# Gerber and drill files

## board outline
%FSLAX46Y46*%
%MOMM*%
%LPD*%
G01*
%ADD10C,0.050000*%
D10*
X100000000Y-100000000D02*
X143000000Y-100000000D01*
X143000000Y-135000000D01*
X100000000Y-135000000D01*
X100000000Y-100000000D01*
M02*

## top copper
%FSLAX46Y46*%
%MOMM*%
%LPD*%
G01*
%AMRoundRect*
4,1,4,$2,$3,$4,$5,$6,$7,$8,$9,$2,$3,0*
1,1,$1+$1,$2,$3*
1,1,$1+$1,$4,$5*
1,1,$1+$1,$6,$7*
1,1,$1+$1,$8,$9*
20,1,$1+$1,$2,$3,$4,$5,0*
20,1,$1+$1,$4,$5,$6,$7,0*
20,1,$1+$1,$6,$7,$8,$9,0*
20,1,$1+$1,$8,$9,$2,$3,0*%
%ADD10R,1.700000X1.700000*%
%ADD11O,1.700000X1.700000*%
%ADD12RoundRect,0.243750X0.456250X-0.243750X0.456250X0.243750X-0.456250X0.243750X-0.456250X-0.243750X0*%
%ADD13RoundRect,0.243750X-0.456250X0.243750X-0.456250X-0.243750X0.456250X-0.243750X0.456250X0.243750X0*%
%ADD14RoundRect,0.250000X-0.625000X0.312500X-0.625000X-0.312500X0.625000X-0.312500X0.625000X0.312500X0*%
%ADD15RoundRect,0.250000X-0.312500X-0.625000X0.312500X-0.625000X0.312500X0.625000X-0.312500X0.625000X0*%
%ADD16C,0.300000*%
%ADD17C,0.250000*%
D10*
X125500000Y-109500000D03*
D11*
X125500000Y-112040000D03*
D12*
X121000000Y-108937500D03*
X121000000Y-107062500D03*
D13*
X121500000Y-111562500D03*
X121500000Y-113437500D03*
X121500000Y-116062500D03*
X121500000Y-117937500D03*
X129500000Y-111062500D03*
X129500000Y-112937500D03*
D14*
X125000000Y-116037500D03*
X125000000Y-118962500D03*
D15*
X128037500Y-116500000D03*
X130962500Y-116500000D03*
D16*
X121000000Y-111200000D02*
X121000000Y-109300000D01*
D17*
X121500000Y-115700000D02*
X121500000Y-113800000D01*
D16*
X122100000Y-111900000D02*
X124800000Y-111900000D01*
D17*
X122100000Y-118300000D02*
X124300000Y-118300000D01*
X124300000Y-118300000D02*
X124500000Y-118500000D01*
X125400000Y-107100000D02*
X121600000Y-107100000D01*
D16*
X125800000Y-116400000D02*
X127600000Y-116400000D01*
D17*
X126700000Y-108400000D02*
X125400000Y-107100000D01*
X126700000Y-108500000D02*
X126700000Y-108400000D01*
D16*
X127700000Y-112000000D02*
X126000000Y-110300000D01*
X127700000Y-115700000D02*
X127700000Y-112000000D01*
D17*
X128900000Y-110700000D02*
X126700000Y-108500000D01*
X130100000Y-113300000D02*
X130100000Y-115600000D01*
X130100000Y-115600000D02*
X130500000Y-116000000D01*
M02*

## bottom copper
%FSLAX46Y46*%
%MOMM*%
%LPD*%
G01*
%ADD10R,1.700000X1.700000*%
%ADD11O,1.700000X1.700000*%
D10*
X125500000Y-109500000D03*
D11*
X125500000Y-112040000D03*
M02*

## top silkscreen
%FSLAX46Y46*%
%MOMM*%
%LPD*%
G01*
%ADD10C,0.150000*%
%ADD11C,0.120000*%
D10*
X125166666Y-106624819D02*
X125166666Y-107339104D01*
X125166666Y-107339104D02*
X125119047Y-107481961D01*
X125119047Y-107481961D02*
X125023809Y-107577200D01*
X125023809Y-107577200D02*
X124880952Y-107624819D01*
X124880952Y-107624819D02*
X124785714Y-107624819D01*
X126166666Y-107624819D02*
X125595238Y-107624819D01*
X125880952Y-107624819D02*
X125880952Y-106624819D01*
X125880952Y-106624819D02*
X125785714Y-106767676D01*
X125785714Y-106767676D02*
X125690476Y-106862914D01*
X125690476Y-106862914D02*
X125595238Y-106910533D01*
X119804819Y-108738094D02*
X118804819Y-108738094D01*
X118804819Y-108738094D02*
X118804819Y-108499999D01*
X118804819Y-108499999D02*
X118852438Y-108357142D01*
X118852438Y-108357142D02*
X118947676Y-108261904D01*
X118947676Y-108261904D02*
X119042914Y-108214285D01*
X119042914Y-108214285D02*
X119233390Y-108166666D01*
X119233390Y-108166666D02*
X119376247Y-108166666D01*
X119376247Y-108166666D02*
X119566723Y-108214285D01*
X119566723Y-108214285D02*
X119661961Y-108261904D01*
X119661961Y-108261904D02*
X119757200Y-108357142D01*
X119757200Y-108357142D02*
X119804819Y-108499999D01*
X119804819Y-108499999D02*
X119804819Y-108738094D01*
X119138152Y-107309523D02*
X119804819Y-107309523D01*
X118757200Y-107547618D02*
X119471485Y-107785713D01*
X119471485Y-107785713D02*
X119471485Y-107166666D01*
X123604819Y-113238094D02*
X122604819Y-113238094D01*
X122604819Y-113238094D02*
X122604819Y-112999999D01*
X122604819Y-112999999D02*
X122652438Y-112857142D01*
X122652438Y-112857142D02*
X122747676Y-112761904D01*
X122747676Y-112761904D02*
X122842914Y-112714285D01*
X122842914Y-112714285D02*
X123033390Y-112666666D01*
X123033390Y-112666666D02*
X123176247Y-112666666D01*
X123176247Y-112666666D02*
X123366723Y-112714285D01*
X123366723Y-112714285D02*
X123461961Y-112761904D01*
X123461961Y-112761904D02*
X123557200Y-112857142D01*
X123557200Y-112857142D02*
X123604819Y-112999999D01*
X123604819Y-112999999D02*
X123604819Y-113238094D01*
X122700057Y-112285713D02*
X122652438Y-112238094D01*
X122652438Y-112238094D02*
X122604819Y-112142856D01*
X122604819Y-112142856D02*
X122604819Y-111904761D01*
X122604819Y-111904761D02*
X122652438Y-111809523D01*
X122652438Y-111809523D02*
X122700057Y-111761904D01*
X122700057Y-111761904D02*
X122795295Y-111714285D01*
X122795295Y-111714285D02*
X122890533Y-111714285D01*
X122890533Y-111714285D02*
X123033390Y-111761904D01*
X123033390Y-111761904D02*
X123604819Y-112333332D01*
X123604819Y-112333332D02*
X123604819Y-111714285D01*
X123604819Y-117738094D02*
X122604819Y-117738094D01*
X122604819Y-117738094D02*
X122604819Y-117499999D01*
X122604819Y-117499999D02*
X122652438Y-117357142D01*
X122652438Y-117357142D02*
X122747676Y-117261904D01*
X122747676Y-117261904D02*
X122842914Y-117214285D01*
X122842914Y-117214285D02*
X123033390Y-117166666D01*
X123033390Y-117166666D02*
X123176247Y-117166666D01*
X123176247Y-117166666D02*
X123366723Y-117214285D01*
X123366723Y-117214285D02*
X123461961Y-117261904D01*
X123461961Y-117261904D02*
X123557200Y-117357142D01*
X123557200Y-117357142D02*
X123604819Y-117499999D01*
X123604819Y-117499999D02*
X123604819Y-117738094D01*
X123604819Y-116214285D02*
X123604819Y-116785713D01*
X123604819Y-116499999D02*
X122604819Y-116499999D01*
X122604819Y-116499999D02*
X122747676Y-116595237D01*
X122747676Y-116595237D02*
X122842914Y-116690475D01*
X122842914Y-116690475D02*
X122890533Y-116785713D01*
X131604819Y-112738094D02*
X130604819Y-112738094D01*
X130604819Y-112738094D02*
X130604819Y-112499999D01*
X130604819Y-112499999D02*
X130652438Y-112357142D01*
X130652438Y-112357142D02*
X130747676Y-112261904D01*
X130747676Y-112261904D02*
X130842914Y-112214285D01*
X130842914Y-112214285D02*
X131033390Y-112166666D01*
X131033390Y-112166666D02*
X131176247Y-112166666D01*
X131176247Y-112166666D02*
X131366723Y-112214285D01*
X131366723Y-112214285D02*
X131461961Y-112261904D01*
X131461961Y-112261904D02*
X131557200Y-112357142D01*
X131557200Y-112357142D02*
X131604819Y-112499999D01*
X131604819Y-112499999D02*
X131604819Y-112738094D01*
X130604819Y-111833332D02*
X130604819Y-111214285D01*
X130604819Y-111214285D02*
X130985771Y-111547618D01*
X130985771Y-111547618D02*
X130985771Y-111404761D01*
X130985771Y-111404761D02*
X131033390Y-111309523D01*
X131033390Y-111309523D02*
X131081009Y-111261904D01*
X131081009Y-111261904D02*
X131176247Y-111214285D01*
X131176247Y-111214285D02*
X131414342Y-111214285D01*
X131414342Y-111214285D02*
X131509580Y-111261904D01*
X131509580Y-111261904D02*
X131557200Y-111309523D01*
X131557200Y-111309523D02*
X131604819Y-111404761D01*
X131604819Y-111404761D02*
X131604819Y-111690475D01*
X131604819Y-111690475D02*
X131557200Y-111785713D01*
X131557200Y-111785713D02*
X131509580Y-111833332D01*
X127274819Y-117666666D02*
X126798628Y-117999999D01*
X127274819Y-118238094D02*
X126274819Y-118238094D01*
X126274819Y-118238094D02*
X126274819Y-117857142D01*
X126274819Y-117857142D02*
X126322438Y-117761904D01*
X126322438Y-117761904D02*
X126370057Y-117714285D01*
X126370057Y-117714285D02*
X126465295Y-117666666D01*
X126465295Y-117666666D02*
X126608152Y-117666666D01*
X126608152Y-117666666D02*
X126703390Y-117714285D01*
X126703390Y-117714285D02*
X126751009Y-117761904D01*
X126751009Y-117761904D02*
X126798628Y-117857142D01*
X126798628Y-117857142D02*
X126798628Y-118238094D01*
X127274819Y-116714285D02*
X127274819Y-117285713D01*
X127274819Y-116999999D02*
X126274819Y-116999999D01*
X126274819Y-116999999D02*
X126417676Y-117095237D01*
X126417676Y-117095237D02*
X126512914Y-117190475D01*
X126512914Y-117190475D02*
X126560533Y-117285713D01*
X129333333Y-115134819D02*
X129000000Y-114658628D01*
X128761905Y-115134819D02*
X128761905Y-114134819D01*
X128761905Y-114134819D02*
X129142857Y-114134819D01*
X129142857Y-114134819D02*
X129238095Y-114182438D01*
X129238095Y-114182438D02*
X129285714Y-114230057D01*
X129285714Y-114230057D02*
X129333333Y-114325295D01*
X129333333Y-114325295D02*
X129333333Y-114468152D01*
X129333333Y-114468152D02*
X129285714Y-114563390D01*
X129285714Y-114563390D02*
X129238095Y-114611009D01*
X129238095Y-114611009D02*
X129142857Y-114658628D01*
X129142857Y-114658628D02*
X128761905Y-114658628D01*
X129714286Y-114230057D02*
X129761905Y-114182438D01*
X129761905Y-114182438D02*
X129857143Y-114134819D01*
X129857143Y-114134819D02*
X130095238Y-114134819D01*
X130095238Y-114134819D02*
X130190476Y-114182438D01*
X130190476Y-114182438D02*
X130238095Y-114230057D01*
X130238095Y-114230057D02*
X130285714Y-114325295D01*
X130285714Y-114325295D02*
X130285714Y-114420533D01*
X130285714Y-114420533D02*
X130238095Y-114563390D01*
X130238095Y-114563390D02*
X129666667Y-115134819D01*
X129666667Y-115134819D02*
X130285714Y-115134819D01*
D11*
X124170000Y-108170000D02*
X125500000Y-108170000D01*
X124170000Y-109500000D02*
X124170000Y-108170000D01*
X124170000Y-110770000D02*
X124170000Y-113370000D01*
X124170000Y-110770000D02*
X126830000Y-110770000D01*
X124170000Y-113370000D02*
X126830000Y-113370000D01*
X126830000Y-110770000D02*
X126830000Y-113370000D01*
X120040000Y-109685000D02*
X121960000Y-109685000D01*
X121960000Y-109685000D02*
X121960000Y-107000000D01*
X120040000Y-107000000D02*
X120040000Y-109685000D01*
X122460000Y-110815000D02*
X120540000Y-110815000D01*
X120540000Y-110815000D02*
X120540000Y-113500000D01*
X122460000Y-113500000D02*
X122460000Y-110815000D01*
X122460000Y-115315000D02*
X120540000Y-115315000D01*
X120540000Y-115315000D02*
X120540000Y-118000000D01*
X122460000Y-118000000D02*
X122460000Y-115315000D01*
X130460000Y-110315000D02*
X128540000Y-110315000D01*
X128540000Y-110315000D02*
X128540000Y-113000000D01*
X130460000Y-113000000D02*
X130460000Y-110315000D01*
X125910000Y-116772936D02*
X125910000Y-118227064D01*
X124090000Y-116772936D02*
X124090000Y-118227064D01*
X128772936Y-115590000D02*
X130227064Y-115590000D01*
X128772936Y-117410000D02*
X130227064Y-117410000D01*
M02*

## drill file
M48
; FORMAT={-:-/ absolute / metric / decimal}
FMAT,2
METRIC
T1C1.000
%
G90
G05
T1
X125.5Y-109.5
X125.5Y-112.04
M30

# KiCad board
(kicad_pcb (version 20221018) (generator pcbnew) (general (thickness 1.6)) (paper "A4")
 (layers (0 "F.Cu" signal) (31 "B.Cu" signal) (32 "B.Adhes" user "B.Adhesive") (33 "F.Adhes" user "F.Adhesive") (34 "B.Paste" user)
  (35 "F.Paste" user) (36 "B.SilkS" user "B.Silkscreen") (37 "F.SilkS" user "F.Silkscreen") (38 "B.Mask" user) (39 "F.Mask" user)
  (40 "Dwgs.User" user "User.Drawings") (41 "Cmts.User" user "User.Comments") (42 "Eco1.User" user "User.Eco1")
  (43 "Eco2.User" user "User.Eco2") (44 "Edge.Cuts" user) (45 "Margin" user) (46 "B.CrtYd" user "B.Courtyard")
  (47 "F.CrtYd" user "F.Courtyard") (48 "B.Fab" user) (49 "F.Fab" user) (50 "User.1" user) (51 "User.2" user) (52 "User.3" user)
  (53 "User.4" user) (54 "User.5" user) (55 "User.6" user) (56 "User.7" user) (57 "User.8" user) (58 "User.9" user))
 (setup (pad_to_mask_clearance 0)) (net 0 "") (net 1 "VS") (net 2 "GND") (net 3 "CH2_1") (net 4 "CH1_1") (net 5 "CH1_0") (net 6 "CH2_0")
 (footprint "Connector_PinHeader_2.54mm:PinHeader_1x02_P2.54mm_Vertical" (layer "F.Cu") (at 125.5 109.5)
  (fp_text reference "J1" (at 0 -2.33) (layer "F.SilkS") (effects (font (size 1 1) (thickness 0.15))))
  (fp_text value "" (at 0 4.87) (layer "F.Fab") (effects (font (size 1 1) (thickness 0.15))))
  (fp_line (start -1.33 -1.33) (end 0 -1.33) (stroke (width 0.12) (type solid)) (layer "F.SilkS"))
  (fp_line (start -1.33 0) (end -1.33 -1.33) (stroke (width 0.12) (type solid)) (layer "F.SilkS"))
  (fp_line (start -1.33 1.27) (end -1.33 3.87) (stroke (width 0.12) (type solid)) (layer "F.SilkS"))
  (fp_line (start -1.33 1.27) (end 1.33 1.27) (stroke (width 0.12) (type solid)) (layer "F.SilkS"))
  (fp_line (start -1.33 3.87) (end 1.33 3.87) (stroke (width 0.12) (type solid)) (layer "F.SilkS"))
  (fp_line (start 1.33 1.27) (end 1.33 3.87) (stroke (width 0.12) (type solid)) (layer "F.SilkS"))
  (pad "1" thru_hole rect (at 0 0) (size 1.7 1.7) (drill 1) (layers "*.Cu" "*.Mask") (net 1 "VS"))
  (pad "2" thru_hole oval (at 0 2.54) (size 1.7 1.7) (drill 1) (layers "*.Cu" "*.Mask") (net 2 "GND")))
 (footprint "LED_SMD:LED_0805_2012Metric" (layer "F.Cu") (at 121 108 90)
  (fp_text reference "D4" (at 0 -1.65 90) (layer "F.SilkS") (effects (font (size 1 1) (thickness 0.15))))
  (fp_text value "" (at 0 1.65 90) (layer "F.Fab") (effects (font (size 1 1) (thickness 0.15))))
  (fp_line (start -1.685 -0.96) (end -1.685 0.96) (stroke (width 0.12) (type solid)) (layer "F.SilkS"))
  (fp_line (start -1.685 0.96) (end 1 0.96) (stroke (width 0.12) (type solid)) (layer "F.SilkS"))
  (fp_line (start 1 -0.96) (end -1.685 -0.96) (stroke (width 0.12) (type solid)) (layer "F.SilkS"))
  (pad "1" smd roundrect (at -0.9375 0 90) (size 0.975 1.4) (layers "F.Cu" "F.Paste" "F.Mask") (roundrect_rratio 0.25) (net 2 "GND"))
  (pad "2" smd roundrect (at 0.9375 0 90) (size 0.975 1.4) (layers "F.Cu" "F.Paste" "F.Mask") (roundrect_rratio 0.25) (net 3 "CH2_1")))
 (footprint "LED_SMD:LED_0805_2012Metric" (layer "F.Cu") (at 121.5 112.5 -90)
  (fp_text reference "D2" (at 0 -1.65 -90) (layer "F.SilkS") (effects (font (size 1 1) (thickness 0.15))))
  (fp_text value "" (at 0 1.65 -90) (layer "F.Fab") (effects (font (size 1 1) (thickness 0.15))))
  (fp_line (start -1.685 -0.96) (end -1.685 0.96) (stroke (width 0.12) (type solid)) (layer "F.SilkS"))
  (fp_line (start -1.685 0.96) (end 1 0.96) (stroke (width 0.12) (type solid)) (layer "F.SilkS"))
  (fp_line (start 1 -0.96) (end -1.685 -0.96) (stroke (width 0.12) (type solid)) (layer "F.SilkS"))
  (pad "1" smd roundrect (at -0.9375 0 270) (size 0.975 1.4) (layers "F.Cu" "F.Paste" "F.Mask") (roundrect_rratio 0.25) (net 2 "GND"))
  (pad "2" smd roundrect (at 0.9375 0 270) (size 0.975 1.4) (layers "F.Cu" "F.Paste" "F.Mask") (roundrect_rratio 0.25) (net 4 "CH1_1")))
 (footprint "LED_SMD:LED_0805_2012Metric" (layer "F.Cu") (at 121.5 117 -90)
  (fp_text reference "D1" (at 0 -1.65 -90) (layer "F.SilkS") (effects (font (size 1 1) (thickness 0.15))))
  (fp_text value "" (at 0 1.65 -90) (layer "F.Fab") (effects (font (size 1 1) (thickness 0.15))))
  (fp_line (start -1.685 -0.96) (end -1.685 0.96) (stroke (width 0.12) (type solid)) (layer "F.SilkS"))
  (fp_line (start -1.685 0.96) (end 1 0.96) (stroke (width 0.12) (type solid)) (layer "F.SilkS"))
  (fp_line (start 1 -0.96) (end -1.685 -0.96) (stroke (width 0.12) (type solid)) (layer "F.SilkS"))
  (pad "1" smd roundrect (at -0.9375 0 270) (size 0.975 1.4) (layers "F.Cu" "F.Paste" "F.Mask") (roundrect_rratio 0.25) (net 4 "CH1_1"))
  (pad "2" smd roundrect (at 0.9375 0 270) (size 0.975 1.4) (layers "F.Cu" "F.Paste" "F.Mask") (roundrect_rratio 0.25) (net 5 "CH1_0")))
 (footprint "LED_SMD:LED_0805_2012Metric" (layer "F.Cu") (at 129.5 112 -90)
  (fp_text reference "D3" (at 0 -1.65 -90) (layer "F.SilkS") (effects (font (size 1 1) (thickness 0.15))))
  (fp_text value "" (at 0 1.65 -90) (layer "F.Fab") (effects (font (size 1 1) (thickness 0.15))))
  (fp_line (start -1.685 -0.96) (end -1.685 0.96) (stroke (width 0.12) (type solid)) (layer "F.SilkS"))
  (fp_line (start -1.685 0.96) (end 1 0.96) (stroke (width 0.12) (type solid)) (layer "F.SilkS"))
  (fp_line (start 1 -0.96) (end -1.685 -0.96) (stroke (width 0.12) (type solid)) (layer "F.SilkS"))
  (pad "1" smd roundrect (at -0.9375 0 270) (size 0.975 1.4) (layers "F.Cu" "F.Paste" "F.Mask") (roundrect_rratio 0.25) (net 3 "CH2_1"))
  (pad "2" smd roundrect (at 0.9375 0 270) (size 0.975 1.4) (layers "F.Cu" "F.Paste" "F.Mask") (roundrect_rratio 0.25) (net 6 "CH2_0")))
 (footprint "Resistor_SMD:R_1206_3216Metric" (layer "F.Cu") (at 125 117.5 -90)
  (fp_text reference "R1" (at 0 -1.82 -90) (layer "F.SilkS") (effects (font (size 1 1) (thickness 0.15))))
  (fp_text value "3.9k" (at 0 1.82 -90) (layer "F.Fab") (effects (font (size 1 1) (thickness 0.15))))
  (fp_line (start -0.727064 -0.91) (end 0.727064 -0.91) (stroke (width 0.12) (type solid)) (layer "F.SilkS"))
  (fp_line (start -0.727064 0.91) (end 0.727064 0.91) (stroke (width 0.12) (type solid)) (layer "F.SilkS"))
  (pad "1" smd roundrect (at -1.4625 0 270) (size 1.125 1.75) (layers "F.Cu" "F.Paste" "F.Mask") (roundrect_rratio 0.222222) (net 1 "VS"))
  (pad "2" smd roundrect (at 1.4625 0 270) (size 1.125 1.75) (layers "F.Cu" "F.Paste" "F.Mask") (roundrect_rratio 0.222222) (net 5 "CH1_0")))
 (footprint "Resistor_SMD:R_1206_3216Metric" (layer "F.Cu") (at 129.5 116.5)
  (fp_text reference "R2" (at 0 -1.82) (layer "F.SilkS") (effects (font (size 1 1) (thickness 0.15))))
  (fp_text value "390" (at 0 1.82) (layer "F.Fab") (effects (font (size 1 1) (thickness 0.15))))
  (fp_line (start -0.727064 -0.91) (end 0.727064 -0.91) (stroke (width 0.12) (type solid)) (layer "F.SilkS"))
  (fp_line (start -0.727064 0.91) (end 0.727064 0.91) (stroke (width 0.12) (type solid)) (layer "F.SilkS"))
  (pad "1" smd roundrect (at -1.4625 0) (size 1.125 1.75) (layers "F.Cu" "F.Paste" "F.Mask") (roundrect_rratio 0.222222) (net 1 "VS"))
  (pad "2" smd roundrect (at 1.4625 0) (size 1.125 1.75) (layers "F.Cu" "F.Paste" "F.Mask") (roundrect_rratio 0.222222) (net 6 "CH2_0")))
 (gr_rect (start 100 100) (end 143 135) (stroke (width 0.05) (type default)) (fill none) (layer "Edge.Cuts"))
 (segment (start 121 111.2) (end 121 109.3) (width 0.3) (layer "F.Cu") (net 2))
 (segment (start 121.5 115.7) (end 121.5 113.8) (width 0.25) (layer "F.Cu") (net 4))
 (segment (start 122.1 111.9) (end 124.8 111.9) (width 0.3) (layer "F.Cu") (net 2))
 (segment (start 122.1 118.3) (end 124.3 118.3) (width 0.25) (layer "F.Cu") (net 5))
 (segment (start 124.3 118.3) (end 124.5 118.5) (width 0.25) (layer "F.Cu") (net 5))
 (segment (start 125.4 107.1) (end 121.6 107.1) (width 0.25) (layer "F.Cu") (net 3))
 (segment (start 125.8 116.4) (end 127.6 116.4) (width 0.3) (layer "F.Cu") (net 1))
 (segment (start 126.7 108.4) (end 125.4 107.1) (width 0.25) (layer "F.Cu") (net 3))
 (segment (start 126.7 108.5) (end 126.7 108.4) (width 0.25) (layer "F.Cu") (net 3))
 (segment (start 127.7 112) (end 126 110.3) (width 0.3) (layer "F.Cu") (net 1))
 (segment (start 127.7 115.7) (end 127.7 112) (width 0.3) (layer "F.Cu") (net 1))
 (segment (start 128.9 110.7) (end 126.7 108.5) (width 0.25) (layer "F.Cu") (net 3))
 (segment (start 130.1 113.3) (end 130.1 115.6) (width 0.25) (layer "F.Cu") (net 6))
 (segment (start 130.1 115.6) (end 130.5 116) (width 0.25) (layer "F.Cu") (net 6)))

